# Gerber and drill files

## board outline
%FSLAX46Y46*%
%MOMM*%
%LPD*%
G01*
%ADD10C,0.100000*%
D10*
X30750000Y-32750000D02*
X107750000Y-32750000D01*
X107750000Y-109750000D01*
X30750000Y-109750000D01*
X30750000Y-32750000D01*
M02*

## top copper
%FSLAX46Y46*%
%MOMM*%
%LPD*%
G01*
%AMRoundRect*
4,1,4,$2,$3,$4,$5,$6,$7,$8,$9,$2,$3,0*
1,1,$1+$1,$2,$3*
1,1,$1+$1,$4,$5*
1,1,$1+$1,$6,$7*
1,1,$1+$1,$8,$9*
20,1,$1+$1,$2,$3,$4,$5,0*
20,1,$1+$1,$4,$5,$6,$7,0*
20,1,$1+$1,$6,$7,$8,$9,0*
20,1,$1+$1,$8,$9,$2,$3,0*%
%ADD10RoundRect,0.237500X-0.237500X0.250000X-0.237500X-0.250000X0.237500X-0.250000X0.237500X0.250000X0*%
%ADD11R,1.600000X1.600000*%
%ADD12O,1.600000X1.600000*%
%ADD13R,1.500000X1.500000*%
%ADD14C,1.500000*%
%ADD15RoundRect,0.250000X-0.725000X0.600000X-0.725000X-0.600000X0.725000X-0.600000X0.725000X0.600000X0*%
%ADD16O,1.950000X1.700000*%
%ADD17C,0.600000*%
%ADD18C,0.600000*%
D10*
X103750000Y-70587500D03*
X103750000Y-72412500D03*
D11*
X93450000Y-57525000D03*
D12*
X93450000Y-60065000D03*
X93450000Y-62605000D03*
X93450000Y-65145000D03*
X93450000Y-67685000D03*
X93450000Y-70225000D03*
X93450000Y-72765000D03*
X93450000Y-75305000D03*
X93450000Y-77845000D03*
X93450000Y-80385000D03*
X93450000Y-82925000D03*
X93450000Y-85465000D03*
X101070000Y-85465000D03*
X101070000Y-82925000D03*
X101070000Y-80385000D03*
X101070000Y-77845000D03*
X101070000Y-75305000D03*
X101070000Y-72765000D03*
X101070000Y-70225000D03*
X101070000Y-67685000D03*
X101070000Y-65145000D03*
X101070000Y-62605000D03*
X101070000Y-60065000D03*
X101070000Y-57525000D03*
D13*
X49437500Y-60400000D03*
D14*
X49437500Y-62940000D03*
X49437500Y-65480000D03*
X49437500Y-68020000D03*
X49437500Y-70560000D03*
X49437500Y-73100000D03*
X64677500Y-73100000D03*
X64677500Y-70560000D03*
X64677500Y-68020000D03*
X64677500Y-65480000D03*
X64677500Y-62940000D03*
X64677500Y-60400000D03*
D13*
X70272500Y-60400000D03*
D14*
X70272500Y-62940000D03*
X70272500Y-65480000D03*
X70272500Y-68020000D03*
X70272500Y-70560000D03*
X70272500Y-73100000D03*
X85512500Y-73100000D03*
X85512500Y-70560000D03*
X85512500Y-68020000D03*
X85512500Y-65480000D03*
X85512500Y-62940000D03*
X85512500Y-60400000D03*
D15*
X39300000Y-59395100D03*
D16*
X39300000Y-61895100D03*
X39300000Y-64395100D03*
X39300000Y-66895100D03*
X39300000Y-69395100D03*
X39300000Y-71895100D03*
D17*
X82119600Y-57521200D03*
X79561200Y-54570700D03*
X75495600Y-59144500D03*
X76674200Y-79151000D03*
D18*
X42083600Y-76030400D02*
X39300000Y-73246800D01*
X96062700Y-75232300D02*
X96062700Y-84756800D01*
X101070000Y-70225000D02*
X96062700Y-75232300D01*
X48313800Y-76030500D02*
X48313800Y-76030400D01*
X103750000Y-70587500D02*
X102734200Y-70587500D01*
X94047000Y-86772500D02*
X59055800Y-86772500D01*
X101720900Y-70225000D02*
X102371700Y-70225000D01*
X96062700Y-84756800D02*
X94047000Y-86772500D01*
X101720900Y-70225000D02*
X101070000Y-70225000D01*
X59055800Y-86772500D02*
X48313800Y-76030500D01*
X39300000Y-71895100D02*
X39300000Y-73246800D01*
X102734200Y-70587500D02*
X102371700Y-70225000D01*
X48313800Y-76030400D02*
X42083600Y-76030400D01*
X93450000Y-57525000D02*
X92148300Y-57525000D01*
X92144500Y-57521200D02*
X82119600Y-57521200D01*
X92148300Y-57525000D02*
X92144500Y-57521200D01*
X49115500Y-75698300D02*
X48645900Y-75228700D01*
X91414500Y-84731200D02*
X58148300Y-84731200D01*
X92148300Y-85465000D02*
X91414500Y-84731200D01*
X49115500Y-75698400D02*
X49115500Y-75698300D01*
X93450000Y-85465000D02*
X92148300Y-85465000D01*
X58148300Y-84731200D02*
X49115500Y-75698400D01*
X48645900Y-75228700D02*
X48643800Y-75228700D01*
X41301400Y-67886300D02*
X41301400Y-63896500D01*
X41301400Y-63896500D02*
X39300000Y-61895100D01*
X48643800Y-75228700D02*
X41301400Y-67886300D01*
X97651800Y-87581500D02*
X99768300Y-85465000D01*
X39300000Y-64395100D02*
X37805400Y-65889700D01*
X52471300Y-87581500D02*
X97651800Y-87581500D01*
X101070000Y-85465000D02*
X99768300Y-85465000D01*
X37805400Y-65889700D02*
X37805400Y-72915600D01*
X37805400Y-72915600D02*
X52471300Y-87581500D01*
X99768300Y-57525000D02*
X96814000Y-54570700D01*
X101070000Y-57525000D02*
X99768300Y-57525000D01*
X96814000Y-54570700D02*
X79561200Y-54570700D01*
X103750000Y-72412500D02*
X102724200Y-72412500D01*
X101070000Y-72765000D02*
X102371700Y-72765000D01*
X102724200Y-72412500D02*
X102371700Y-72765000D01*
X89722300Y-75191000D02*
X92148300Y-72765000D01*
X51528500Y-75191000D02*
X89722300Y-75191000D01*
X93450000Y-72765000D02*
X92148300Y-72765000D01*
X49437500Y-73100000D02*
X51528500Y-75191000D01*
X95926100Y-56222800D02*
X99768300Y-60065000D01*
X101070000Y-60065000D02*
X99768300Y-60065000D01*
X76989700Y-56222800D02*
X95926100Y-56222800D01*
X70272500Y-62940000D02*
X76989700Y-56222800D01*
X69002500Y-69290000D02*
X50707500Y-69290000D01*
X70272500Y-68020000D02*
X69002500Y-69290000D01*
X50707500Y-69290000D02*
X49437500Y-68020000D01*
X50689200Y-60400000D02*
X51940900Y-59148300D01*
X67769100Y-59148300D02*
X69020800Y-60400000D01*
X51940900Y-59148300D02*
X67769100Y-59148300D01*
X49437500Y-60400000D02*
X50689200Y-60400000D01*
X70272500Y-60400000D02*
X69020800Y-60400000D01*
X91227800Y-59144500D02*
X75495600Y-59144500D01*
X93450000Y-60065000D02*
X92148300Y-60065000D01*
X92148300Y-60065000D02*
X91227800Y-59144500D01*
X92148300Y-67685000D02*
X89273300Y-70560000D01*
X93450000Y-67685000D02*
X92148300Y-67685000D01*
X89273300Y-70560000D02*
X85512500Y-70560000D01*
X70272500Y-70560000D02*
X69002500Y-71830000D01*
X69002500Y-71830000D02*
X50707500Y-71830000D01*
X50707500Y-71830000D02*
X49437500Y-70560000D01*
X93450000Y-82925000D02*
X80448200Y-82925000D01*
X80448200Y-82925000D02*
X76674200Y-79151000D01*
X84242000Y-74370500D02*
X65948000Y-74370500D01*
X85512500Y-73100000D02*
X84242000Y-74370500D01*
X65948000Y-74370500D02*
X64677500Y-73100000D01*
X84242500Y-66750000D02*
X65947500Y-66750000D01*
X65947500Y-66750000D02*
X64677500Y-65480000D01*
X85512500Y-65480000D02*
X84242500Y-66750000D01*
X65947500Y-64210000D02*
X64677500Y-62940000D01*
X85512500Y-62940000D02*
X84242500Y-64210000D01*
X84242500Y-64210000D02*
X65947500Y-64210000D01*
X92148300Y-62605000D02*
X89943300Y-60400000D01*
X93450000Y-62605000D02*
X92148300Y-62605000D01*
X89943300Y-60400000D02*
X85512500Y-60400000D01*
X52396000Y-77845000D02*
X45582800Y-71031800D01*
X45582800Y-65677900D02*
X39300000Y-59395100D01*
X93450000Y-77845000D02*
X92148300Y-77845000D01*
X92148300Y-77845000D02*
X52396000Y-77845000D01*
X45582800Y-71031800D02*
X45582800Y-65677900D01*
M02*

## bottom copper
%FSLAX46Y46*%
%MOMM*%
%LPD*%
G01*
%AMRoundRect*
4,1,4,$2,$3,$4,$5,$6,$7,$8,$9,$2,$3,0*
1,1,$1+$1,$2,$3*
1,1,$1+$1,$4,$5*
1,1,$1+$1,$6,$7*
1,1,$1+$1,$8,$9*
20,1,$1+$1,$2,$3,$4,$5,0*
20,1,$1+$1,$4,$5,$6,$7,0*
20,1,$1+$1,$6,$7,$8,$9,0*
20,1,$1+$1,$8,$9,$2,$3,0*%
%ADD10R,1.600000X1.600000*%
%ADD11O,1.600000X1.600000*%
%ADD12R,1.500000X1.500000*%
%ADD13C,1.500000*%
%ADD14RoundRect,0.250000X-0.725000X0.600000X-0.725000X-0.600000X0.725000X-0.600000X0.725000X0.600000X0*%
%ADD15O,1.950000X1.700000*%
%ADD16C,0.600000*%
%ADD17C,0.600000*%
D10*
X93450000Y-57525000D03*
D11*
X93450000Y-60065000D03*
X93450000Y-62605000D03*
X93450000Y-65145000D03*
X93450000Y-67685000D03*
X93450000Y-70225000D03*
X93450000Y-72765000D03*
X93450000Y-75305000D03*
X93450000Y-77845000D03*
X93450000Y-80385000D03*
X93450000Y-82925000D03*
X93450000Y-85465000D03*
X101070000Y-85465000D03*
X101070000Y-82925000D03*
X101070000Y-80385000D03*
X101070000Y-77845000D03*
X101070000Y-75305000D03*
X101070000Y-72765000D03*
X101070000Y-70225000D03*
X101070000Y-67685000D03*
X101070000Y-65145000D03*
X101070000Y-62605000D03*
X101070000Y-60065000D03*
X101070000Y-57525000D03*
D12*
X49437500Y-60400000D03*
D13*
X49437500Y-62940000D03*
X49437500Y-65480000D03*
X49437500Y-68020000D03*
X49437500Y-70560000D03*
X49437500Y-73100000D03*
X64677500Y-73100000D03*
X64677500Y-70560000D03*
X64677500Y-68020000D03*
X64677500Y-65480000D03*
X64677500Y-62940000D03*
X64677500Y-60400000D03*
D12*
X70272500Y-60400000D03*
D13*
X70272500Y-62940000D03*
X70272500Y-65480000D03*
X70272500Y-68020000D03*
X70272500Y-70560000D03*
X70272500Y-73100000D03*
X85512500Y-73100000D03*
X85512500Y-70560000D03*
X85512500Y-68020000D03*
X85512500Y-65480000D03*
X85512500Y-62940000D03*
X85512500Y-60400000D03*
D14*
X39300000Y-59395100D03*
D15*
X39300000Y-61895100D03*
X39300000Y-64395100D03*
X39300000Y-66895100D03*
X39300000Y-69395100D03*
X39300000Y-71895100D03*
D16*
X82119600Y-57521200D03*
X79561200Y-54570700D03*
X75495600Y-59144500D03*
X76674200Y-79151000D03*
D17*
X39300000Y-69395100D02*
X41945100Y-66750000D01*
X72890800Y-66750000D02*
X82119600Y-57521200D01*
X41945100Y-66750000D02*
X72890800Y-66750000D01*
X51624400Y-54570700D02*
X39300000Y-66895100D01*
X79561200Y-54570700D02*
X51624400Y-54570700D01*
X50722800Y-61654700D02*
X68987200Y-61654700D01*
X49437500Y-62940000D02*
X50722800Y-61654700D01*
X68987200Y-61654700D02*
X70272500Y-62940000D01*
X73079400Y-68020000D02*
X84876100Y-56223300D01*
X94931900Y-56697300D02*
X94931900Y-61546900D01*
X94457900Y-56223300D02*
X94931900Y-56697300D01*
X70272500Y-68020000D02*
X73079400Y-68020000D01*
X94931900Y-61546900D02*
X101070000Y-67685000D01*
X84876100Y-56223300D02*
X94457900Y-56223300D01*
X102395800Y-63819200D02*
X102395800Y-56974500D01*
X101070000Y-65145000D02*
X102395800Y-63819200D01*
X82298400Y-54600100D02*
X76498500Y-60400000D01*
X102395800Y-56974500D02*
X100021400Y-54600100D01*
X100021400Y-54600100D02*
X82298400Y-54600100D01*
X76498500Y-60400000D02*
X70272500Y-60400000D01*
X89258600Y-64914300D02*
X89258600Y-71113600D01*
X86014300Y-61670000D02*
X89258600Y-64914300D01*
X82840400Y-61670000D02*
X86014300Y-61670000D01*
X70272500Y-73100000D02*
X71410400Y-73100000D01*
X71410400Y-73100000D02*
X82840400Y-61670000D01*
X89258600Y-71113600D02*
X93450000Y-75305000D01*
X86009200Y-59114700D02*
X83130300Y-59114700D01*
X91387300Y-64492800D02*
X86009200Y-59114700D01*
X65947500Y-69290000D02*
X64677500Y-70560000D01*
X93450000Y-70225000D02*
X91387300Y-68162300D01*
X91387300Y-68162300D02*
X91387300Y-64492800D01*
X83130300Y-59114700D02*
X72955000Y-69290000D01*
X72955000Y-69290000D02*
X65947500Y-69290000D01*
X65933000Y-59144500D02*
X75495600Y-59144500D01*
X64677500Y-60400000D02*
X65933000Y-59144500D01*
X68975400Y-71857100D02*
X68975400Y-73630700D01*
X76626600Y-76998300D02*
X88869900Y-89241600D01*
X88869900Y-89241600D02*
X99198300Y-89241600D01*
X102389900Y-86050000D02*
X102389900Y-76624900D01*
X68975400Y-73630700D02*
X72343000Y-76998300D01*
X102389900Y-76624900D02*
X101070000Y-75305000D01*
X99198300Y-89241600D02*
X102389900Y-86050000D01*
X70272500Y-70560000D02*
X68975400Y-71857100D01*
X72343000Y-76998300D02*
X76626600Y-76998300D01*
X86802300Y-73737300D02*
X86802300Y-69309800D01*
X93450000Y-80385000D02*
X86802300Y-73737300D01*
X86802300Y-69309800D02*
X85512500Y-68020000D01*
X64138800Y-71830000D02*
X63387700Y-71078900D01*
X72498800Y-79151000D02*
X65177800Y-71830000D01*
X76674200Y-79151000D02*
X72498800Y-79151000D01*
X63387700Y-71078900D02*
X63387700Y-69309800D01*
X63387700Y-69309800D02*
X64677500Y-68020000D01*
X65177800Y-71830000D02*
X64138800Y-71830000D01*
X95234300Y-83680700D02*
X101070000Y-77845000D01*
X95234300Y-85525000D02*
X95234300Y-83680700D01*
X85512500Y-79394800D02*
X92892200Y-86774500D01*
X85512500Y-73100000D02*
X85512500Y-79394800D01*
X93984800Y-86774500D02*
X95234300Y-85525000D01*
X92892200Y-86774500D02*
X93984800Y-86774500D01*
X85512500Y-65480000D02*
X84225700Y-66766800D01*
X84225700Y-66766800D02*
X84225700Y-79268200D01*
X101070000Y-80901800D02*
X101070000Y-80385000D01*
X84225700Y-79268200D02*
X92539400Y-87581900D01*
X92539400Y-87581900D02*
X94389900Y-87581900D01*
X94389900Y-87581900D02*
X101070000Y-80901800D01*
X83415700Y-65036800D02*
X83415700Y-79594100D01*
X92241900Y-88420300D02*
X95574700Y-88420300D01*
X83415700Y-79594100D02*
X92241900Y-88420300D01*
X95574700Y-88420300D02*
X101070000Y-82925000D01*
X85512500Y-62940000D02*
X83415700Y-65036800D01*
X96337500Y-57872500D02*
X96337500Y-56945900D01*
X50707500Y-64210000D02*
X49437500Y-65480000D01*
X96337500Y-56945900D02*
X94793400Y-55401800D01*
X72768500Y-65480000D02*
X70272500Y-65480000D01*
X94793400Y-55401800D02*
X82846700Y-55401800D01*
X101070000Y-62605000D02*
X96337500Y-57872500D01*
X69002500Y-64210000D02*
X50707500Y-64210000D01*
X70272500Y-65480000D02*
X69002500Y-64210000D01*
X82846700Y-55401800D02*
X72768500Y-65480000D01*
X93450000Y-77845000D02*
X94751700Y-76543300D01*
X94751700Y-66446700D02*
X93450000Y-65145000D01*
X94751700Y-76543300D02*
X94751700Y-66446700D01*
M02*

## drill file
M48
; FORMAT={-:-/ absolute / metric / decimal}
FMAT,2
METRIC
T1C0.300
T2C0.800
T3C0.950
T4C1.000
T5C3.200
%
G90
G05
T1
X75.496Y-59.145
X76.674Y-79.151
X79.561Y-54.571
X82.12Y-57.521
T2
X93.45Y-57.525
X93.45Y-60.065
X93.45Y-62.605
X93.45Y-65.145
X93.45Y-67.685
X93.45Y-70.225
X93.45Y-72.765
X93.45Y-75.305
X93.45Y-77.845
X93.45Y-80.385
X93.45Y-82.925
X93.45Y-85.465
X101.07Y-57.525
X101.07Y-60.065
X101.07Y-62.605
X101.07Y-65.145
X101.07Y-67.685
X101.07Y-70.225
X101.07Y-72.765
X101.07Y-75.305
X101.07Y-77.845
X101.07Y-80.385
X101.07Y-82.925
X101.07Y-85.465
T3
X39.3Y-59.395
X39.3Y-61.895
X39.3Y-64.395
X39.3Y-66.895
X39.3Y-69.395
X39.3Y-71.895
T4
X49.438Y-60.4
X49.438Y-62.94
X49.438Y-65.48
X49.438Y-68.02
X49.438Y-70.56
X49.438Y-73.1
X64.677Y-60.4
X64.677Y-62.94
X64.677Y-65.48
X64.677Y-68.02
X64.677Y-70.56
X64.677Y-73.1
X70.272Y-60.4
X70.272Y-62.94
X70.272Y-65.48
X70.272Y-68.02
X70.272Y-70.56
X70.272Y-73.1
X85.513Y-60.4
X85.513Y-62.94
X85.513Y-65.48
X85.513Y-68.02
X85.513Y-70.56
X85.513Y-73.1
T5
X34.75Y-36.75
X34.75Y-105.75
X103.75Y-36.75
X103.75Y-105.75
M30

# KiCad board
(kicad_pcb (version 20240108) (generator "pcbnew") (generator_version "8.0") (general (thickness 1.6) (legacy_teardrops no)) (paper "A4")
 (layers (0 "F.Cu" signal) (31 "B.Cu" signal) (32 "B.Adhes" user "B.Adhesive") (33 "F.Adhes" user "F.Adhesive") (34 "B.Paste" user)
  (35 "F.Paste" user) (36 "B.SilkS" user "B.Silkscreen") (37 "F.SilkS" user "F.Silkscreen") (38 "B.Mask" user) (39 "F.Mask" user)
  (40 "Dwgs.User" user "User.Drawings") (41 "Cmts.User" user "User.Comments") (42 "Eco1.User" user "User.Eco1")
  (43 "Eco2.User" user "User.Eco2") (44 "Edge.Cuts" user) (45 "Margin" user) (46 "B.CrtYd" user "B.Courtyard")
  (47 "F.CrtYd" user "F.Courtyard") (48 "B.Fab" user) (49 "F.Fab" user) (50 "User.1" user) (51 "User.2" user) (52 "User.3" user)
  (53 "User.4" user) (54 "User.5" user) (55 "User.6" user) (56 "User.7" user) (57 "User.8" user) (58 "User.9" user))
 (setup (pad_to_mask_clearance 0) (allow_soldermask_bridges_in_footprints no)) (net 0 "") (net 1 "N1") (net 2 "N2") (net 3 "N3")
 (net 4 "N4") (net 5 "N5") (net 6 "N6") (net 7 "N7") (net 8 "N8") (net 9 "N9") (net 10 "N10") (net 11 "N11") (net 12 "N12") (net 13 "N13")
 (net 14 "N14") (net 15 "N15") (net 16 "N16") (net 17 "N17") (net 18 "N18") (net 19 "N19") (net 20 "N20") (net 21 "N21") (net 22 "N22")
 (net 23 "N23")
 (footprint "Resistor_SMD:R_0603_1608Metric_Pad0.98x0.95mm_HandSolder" (layer "F.Cu") (at 103.75 71.5 -90)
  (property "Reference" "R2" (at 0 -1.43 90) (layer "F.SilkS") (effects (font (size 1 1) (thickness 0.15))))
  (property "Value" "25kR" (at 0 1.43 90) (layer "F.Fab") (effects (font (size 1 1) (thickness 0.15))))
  (pad "1" smd roundrect (at -0.9125 0 270) (size 0.975 0.95) (layers "F.Cu" "F.Paste" "F.Mask") (roundrect_rratio 0.25) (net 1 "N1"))
  (pad "2" smd roundrect (at 0.9125 0 270) (size 0.975 0.95) (layers "F.Cu" "F.Paste" "F.Mask") (roundrect_rratio 0.25) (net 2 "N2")))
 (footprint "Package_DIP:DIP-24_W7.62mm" (layer "F.Cu") (at 93.45 57.525)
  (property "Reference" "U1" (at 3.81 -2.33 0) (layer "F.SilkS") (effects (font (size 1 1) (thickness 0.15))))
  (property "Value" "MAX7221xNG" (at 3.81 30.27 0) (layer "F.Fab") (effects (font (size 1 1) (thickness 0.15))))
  (pad "1" thru_hole rect (at 0 0) (size 1.6 1.6) (drill 0.8) (layers "*.Cu" "*.Mask") (remove_unused_layers no) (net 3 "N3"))
  (pad "2" thru_hole oval (at 0 2.54) (size 1.6 1.6) (drill 0.8) (layers "*.Cu" "*.Mask") (remove_unused_layers no) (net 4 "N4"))
  (pad "3" thru_hole oval (at 0 5.08) (size 1.6 1.6) (drill 0.8) (layers "*.Cu" "*.Mask") (remove_unused_layers no) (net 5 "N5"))
  (pad "4" thru_hole oval (at 0 7.62) (size 1.6 1.6) (drill 0.8) (layers "*.Cu" "*.Mask") (remove_unused_layers no) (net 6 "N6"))
  (pad "5" thru_hole oval (at 0 10.16) (size 1.6 1.6) (drill 0.8) (layers "*.Cu" "*.Mask") (remove_unused_layers no) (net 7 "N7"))
  (pad "6" thru_hole oval (at 0 12.7) (size 1.6 1.6) (drill 0.8) (layers "*.Cu" "*.Mask") (remove_unused_layers no) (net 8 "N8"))
  (pad "7" thru_hole oval (at 0 15.24) (size 1.6 1.6) (drill 0.8) (layers "*.Cu" "*.Mask") (remove_unused_layers no) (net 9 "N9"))
  (pad "8" thru_hole oval (at 0 17.78) (size 1.6 1.6) (drill 0.8) (layers "*.Cu" "*.Mask") (remove_unused_layers no) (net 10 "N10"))
  (pad "9" thru_hole oval (at 0 20.32) (size 1.6 1.6) (drill 0.8) (layers "*.Cu" "*.Mask") (remove_unused_layers no) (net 6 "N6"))
  (pad "10" thru_hole oval (at 0 22.86) (size 1.6 1.6) (drill 0.8) (layers "*.Cu" "*.Mask") (remove_unused_layers no) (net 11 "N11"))
  (pad "11" thru_hole oval (at 0 25.4) (size 1.6 1.6) (drill 0.8) (layers "*.Cu" "*.Mask") (remove_unused_layers no) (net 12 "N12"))
  (pad "12" thru_hole oval (at 0 27.94) (size 1.6 1.6) (drill 0.8) (layers "*.Cu" "*.Mask") (remove_unused_layers no) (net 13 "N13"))
  (pad "13" thru_hole oval (at 7.62 27.94) (size 1.6 1.6) (drill 0.8) (layers "*.Cu" "*.Mask") (remove_unused_layers no) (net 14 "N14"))
  (pad "14" thru_hole oval (at 7.62 25.4) (size 1.6 1.6) (drill 0.8) (layers "*.Cu" "*.Mask") (remove_unused_layers no) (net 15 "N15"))
  (pad "15" thru_hole oval (at 7.62 22.86) (size 1.6 1.6) (drill 0.8) (layers "*.Cu" "*.Mask") (remove_unused_layers no) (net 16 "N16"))
  (pad "16" thru_hole oval (at 7.62 20.32) (size 1.6 1.6) (drill 0.8) (layers "*.Cu" "*.Mask") (remove_unused_layers no) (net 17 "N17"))
  (pad "17" thru_hole oval (at 7.62 17.78) (size 1.6 1.6) (drill 0.8) (layers "*.Cu" "*.Mask") (remove_unused_layers no) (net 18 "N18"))
  (pad "18" thru_hole oval (at 7.62 15.24) (size 1.6 1.6) (drill 0.8) (layers "*.Cu" "*.Mask") (remove_unused_layers no) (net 2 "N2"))
  (pad "19" thru_hole oval (at 7.62 12.7) (size 1.6 1.6) (drill 0.8) (layers "*.Cu" "*.Mask") (remove_unused_layers no) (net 1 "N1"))
  (pad "20" thru_hole oval (at 7.62 10.16) (size 1.6 1.6) (drill 0.8) (layers "*.Cu" "*.Mask") (remove_unused_layers no) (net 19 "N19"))
  (pad "21" thru_hole oval (at 7.62 7.62) (size 1.6 1.6) (drill 0.8) (layers "*.Cu" "*.Mask") (remove_unused_layers no) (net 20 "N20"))
  (pad "22" thru_hole oval (at 7.62 5.08) (size 1.6 1.6) (drill 0.8) (layers "*.Cu" "*.Mask") (remove_unused_layers no) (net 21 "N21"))
  (pad "23" thru_hole oval (at 7.62 2.54) (size 1.6 1.6) (drill 0.8) (layers "*.Cu" "*.Mask") (remove_unused_layers no) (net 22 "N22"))
  (pad "24" thru_hole oval (at 7.62 0) (size 1.6 1.6) (drill 0.8) (layers "*.Cu" "*.Mask") (remove_unused_layers no) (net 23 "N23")))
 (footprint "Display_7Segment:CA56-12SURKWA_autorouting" (layer "F.Cu") (at 49.4375 60.4)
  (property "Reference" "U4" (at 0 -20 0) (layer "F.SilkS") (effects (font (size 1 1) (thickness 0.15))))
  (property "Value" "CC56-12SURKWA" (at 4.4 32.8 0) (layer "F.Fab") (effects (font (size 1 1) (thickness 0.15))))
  (pad "1" thru_hole rect (at 0 0) (size 1.5 1.5) (drill 1) (layers "*.Cu" "*.Mask") (remove_unused_layers no) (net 20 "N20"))
  (pad "2" thru_hole circle (at 0 2.54) (size 1.5 1.5) (drill 1) (layers "*.Cu" "*.Mask") (remove_unused_layers no) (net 22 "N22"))
  (pad "3" thru_hole circle (at 0 5.08) (size 1.5 1.5) (drill 1) (layers "*.Cu" "*.Mask") (remove_unused_layers no) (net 21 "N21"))
  (pad "4" thru_hole circle (at 0 7.62) (size 1.5 1.5) (drill 1) (layers "*.Cu" "*.Mask") (remove_unused_layers no) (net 19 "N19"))
  (pad "5" thru_hole circle (at 0 10.16) (size 1.5 1.5) (drill 1) (layers "*.Cu" "*.Mask") (remove_unused_layers no) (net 18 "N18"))
  (pad "6" thru_hole circle (at 0 12.7) (size 1.5 1.5) (drill 1) (layers "*.Cu" "*.Mask") (remove_unused_layers no) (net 9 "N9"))
  (pad "7" thru_hole circle (at 15.24 12.7) (size 1.5 1.5) (drill 1) (layers "*.Cu" "*.Mask") (remove_unused_layers no) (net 17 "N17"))
  (pad "8" thru_hole circle (at 15.24 10.16) (size 1.5 1.5) (drill 1) (layers "*.Cu" "*.Mask") (remove_unused_layers no) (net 8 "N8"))
  (pad "9" thru_hole circle (at 15.24 7.62) (size 1.5 1.5) (drill 1) (layers "*.Cu" "*.Mask") (remove_unused_layers no) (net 12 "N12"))
  (pad "10" thru_hole circle (at 15.24 5.08) (size 1.5 1.5) (drill 1) (layers "*.Cu" "*.Mask") (remove_unused_layers no) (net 16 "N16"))
  (pad "11" thru_hole circle (at 15.24 2.54) (size 1.5 1.5) (drill 1) (layers "*.Cu" "*.Mask") (remove_unused_layers no) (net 15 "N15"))
  (pad "12" thru_hole circle (at 15.24 0) (size 1.5 1.5) (drill 1) (layers "*.Cu" "*.Mask") (remove_unused_layers no) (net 4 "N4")))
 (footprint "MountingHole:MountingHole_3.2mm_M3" (layer "F.Cu") (at 34.75 36.75)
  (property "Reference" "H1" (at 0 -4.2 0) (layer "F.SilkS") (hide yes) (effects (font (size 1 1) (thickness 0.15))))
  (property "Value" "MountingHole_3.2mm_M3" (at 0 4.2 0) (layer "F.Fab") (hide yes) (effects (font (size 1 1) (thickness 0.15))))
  (pad "" np_thru_hole circle (at 0 0) (size 3.2 3.2) (drill 3.2) (layers "*.Cu" "*.Mask")))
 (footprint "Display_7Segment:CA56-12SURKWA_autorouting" (layer "F.Cu") (at 70.2725 60.4)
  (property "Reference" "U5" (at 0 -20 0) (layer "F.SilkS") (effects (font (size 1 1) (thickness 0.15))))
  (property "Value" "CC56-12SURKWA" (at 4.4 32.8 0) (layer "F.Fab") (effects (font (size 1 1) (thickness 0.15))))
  (pad "1" thru_hole rect (at 0 0) (size 1.5 1.5) (drill 1) (layers "*.Cu" "*.Mask") (remove_unused_layers no) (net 20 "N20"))
  (pad "2" thru_hole circle (at 0 2.54) (size 1.5 1.5) (drill 1) (layers "*.Cu" "*.Mask") (remove_unused_layers no) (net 22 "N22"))
  (pad "3" thru_hole circle (at 0 5.08) (size 1.5 1.5) (drill 1) (layers "*.Cu" "*.Mask") (remove_unused_layers no) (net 21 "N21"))
  (pad "4" thru_hole circle (at 0 7.62) (size 1.5 1.5) (drill 1) (layers "*.Cu" "*.Mask") (remove_unused_layers no) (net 19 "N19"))
  (pad "5" thru_hole circle (at 0 10.16) (size 1.5 1.5) (drill 1) (layers "*.Cu" "*.Mask") (remove_unused_layers no) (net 18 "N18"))
  (pad "6" thru_hole circle (at 0 12.7) (size 1.5 1.5) (drill 1) (layers "*.Cu" "*.Mask") (remove_unused_layers no) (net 10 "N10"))
  (pad "7" thru_hole circle (at 15.24 12.7) (size 1.5 1.5) (drill 1) (layers "*.Cu" "*.Mask") (remove_unused_layers no) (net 17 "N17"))
  (pad "8" thru_hole circle (at 15.24 10.16) (size 1.5 1.5) (drill 1) (layers "*.Cu" "*.Mask") (remove_unused_layers no) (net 7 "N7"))
  (pad "9" thru_hole circle (at 15.24 7.62) (size 1.5 1.5) (drill 1) (layers "*.Cu" "*.Mask") (remove_unused_layers no) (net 11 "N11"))
  (pad "10" thru_hole circle (at 15.24 5.08) (size 1.5 1.5) (drill 1) (layers "*.Cu" "*.Mask") (remove_unused_layers no) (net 16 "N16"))
  (pad "11" thru_hole circle (at 15.24 2.54) (size 1.5 1.5) (drill 1) (layers "*.Cu" "*.Mask") (remove_unused_layers no) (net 15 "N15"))
  (pad "12" thru_hole circle (at 15.24 0) (size 1.5 1.5) (drill 1) (layers "*.Cu" "*.Mask") (remove_unused_layers no) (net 5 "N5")))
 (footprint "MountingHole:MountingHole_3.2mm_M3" (layer "F.Cu") (at 103.75 36.75)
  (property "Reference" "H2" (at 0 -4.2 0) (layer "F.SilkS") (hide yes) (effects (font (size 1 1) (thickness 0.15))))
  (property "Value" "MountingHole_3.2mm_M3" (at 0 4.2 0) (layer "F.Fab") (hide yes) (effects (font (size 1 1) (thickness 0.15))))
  (pad "" np_thru_hole circle (at 0 0) (size 3.2 3.2) (drill 3.2) (layers "F&B.Cu" "*.Mask")))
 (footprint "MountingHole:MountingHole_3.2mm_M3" (layer "F.Cu") (at 34.75 105.75)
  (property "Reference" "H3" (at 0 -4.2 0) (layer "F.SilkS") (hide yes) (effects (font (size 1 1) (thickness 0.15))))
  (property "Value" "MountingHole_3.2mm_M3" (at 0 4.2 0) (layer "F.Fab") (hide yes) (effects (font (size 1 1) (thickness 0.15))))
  (pad "" np_thru_hole circle (at 0 0) (size 3.2 3.2) (drill 3.2) (layers "F&B.Cu" "*.Mask")))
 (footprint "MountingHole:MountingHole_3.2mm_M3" (layer "F.Cu") (at 103.75 105.75)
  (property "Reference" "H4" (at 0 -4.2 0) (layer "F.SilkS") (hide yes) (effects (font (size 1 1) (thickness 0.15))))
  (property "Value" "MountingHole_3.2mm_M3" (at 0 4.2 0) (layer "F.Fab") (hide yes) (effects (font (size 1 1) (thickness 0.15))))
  (pad "" np_thru_hole circle (at 0 0) (size 3.2 3.2) (drill 3.2) (layers "F&B.Cu" "*.Mask")))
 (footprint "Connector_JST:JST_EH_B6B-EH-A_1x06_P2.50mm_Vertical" (layer "F.Cu") (at 39.3 59.3951 -90)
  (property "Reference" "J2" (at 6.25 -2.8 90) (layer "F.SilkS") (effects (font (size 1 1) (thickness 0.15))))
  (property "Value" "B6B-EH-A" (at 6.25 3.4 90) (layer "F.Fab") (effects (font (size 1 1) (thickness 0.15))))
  (pad "1" thru_hole roundrect (at 0 0 270) (size 1.7 1.95) (drill 0.95) (layers "*.Cu" "*.Mask") (remove_unused_layers no)
   (roundrect_rratio 0.147059) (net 6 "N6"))
  (pad "2" thru_hole oval (at 2.5 0 270) (size 1.7 1.95) (drill 0.95) (layers "*.Cu" "*.Mask") (remove_unused_layers no) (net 13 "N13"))
  (pad "3" thru_hole oval (at 5 0 270) (size 1.7 1.95) (drill 0.95) (layers "*.Cu" "*.Mask") (remove_unused_layers no) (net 14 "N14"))
  (pad "4" thru_hole oval (at 7.5 0 270) (size 1.7 1.95) (drill 0.95) (layers "*.Cu" "*.Mask") (remove_unused_layers no) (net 23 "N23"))
  (pad "5" thru_hole oval (at 10 0 270) (size 1.7 1.95) (drill 0.95) (layers "*.Cu" "*.Mask") (remove_unused_layers no) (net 3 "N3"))
  (pad "6" thru_hole oval (at 12.5 0 270) (size 1.7 1.95) (drill 0.95) (layers "*.Cu" "*.Mask") (remove_unused_layers no) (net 1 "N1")))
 (gr_rect (start 30.75 32.75) (end 107.75 109.75) (stroke (width 0.1) (type default)) (fill none) (layer "Edge.Cuts"))
 (segment (start 42.0836 76.0304) (end 39.3 73.2468) (width 0.6) (layer "F.Cu") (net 1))
 (segment (start 96.0627 75.2323) (end 96.0627 84.7568) (width 0.6) (layer "F.Cu") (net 1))
 (segment (start 101.07 70.225) (end 96.0627 75.2323) (width 0.6) (layer "F.Cu") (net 1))
 (segment (start 48.3138 76.0305) (end 48.3138 76.0304) (width 0.6) (layer "F.Cu") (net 1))
 (segment (start 103.75 70.5875) (end 102.7342 70.5875) (width 0.6) (layer "F.Cu") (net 1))
 (segment (start 94.047 86.7725) (end 59.0558 86.7725) (width 0.6) (layer "F.Cu") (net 1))
 (segment (start 101.7209 70.225) (end 102.3717 70.225) (width 0.6) (layer "F.Cu") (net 1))
 (segment (start 96.0627 84.7568) (end 94.047 86.7725) (width 0.6) (layer "F.Cu") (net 1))
 (segment (start 101.7209 70.225) (end 101.07 70.225) (width 0.6) (layer "F.Cu") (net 1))
 (segment (start 59.0558 86.7725) (end 48.3138 76.0305) (width 0.6) (layer "F.Cu") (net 1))
 (segment (start 39.3 71.8951) (end 39.3 73.2468) (width 0.6) (layer "F.Cu") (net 1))
 (segment (start 102.7342 70.5875) (end 102.3717 70.225) (width 0.6) (layer "F.Cu") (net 1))
 (segment (start 48.3138 76.0304) (end 42.0836 76.0304) (width 0.6) (layer "F.Cu") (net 1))
 (segment (start 93.45 57.525) (end 92.1483 57.525) (width 0.6) (layer "F.Cu") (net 3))
 (segment (start 92.1445 57.5212) (end 82.1196 57.5212) (width 0.6) (layer "F.Cu") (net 3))
 (segment (start 92.1483 57.525) (end 92.1445 57.5212) (width 0.6) (layer "F.Cu") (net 3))
 (via (at 82.1196 57.5212) (size 0.6) (drill 0.3) (layers "F.Cu" "B.Cu") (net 3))
 (segment (start 39.3 69.3951) (end 41.9451 66.75) (width 0.6) (layer "B.Cu") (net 3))
 (segment (start 72.8908 66.75) (end 82.1196 57.5212) (width 0.6) (layer "B.Cu") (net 3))
 (segment (start 41.9451 66.75) (end 72.8908 66.75) (width 0.6) (layer "B.Cu") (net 3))
 (segment (start 49.1155 75.6983) (end 48.6459 75.2287) (width 0.6) (layer "F.Cu") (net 13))
 (segment (start 91.4145 84.7312) (end 58.1483 84.7312) (width 0.6) (layer "F.Cu") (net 13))
 (segment (start 92.1483 85.465) (end 91.4145 84.7312) (width 0.6) (layer "F.Cu") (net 13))
 (segment (start 49.1155 75.6984) (end 49.1155 75.6983) (width 0.6) (layer "F.Cu") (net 13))
 (segment (start 93.45 85.465) (end 92.1483 85.465) (width 0.6) (layer "F.Cu") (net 13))
 (segment (start 58.1483 84.7312) (end 49.1155 75.6984) (width 0.6) (layer "F.Cu") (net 13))
 (segment (start 48.6459 75.2287) (end 48.6438 75.2287) (width 0.6) (layer "F.Cu") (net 13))
 (segment (start 41.3014 67.8863) (end 41.3014 63.8965) (width 0.6) (layer "F.Cu") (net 13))
 (segment (start 41.3014 63.8965) (end 39.3 61.8951) (width 0.6) (layer "F.Cu") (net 13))
 (segment (start 48.6438 75.2287) (end 41.3014 67.8863) (width 0.6) (layer "F.Cu") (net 13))
 (segment (start 97.6518 87.5815) (end 99.7683 85.465) (width 0.6) (layer "F.Cu") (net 14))
 (segment (start 39.3 64.3951) (end 37.8054 65.8897) (width 0.6) (layer "F.Cu") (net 14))
 (segment (start 52.4713 87.5815) (end 97.6518 87.5815) (width 0.6) (layer "F.Cu") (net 14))
 (segment (start 101.07 85.465) (end 99.7683 85.465) (width 0.6) (layer "F.Cu") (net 14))
 (segment (start 37.8054 65.8897) (end 37.8054 72.9156) (width 0.6) (layer "F.Cu") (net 14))
 (segment (start 37.8054 72.9156) (end 52.4713 87.5815) (width 0.6) (layer "F.Cu") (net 14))
 (segment (start 99.7683 57.525) (end 96.814 54.5707) (width 0.6) (layer "F.Cu") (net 23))
 (segment (start 101.07 57.525) (end 99.7683 57.525) (width 0.6) (layer "F.Cu") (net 23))
 (segment (start 96.814 54.5707) (end 79.5612 54.5707) (width 0.6) (layer "F.Cu") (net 23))
 (via (at 79.5612 54.5707) (size 0.6) (drill 0.3) (layers "F.Cu" "B.Cu") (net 23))
 (segment (start 51.6244 54.5707) (end 39.3 66.8951) (width 0.6) (layer "B.Cu") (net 23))
 (segment (start 79.5612 54.5707) (end 51.6244 54.5707) (width 0.6) (layer "B.Cu") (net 23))
 (segment (start 103.75 72.4125) (end 102.7242 72.4125) (width 0.6) (layer "F.Cu") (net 2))
 (segment (start 101.07 72.765) (end 102.3717 72.765) (width 0.6) (layer "F.Cu") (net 2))
 (segment (start 102.7242 72.4125) (end 102.3717 72.765) (width 0.6) (layer "F.Cu") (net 2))
 (segment (start 89.7223 75.191) (end 92.1483 72.765) (width 0.6) (layer "F.Cu") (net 9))
 (segment (start 51.5285 75.191) (end 89.7223 75.191) (width 0.6) (layer "F.Cu") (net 9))
 (segment (start 93.45 72.765) (end 92.1483 72.765) (width 0.6) (layer "F.Cu") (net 9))
 (segment (start 49.4375 73.1) (end 51.5285 75.191) (width 0.6) (layer "F.Cu") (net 9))
 (segment (start 95.9261 56.2228) (end 99.7683 60.065) (width 0.6) (layer "F.Cu") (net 22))
 (segment (start 101.07 60.065) (end 99.7683 60.065) (width 0.6) (layer "F.Cu") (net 22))
 (segment (start 76.9897 56.2228) (end 95.9261 56.2228) (width 0.6) (layer "F.Cu") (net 22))
 (segment (start 70.2725 62.94) (end 76.9897 56.2228) (width 0.6) (layer "F.Cu") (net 22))
 (segment (start 50.7228 61.6547) (end 68.9872 61.6547) (width 0.6) (layer "B.Cu") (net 22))
 (segment (start 49.4375 62.94) (end 50.7228 61.6547) (width 0.6) (layer "B.Cu") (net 22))
 (segment (start 68.9872 61.6547) (end 70.2725 62.94) (width 0.6) (layer "B.Cu") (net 22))
 (segment (start 69.0025 69.29) (end 50.7075 69.29) (width 0.6) (layer "F.Cu") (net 19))
 (segment (start 70.2725 68.02) (end 69.0025 69.29) (width 0.6) (layer "F.Cu") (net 19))
 (segment (start 50.7075 69.29) (end 49.4375 68.02) (width 0.6) (layer "F.Cu") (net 19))
 (segment (start 73.0794 68.02) (end 84.8761 56.2233) (width 0.6) (layer "B.Cu") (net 19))
 (segment (start 94.9319 56.6973) (end 94.9319 61.5469) (width 0.6) (layer "B.Cu") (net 19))
 (segment (start 94.4579 56.2233) (end 94.9319 56.6973) (width 0.6) (layer "B.Cu") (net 19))
 (segment (start 70.2725 68.02) (end 73.0794 68.02) (width 0.6) (layer "B.Cu") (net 19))
 (segment (start 94.9319 61.5469) (end 101.07 67.685) (width 0.6) (layer "B.Cu") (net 19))
 (segment (start 84.8761 56.2233) (end 94.4579 56.2233) (width 0.6) (layer "B.Cu") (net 19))
 (segment (start 50.6892 60.4) (end 51.9409 59.1483) (width 0.6) (layer "F.Cu") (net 20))
 (segment (start 67.7691 59.1483) (end 69.0208 60.4) (width 0.6) (layer "F.Cu") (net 20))
 (segment (start 51.9409 59.1483) (end 67.7691 59.1483) (width 0.6) (layer "F.Cu") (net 20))
 (segment (start 49.4375 60.4) (end 50.6892 60.4) (width 0.6) (layer "F.Cu") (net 20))
 (segment (start 70.2725 60.4) (end 69.0208 60.4) (width 0.6) (layer "F.Cu") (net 20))
 (segment (start 102.3958 63.8192) (end 102.3958 56.9745) (width 0.6) (layer "B.Cu") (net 20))
 (segment (start 101.07 65.145) (end 102.3958 63.8192) (width 0.6) (layer "B.Cu") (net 20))
 (segment (start 82.2984 54.6001) (end 76.4985 60.4) (width 0.6) (layer "B.Cu") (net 20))
 (segment (start 102.3958 56.9745) (end 100.0214 54.6001) (width 0.6) (layer "B.Cu") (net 20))
 (segment (start 100.0214 54.6001) (end 82.2984 54.6001) (width 0.6) (layer "B.Cu") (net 20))
 (segment (start 76.4985 60.4) (end 70.2725 60.4) (width 0.6) (layer "B.Cu") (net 20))
 (segment (start 89.2586 64.9143) (end 89.2586 71.1136) (width 0.6) (layer "B.Cu") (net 10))
 (segment (start 86.0143 61.67) (end 89.2586 64.9143) (width 0.6) (layer "B.Cu") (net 10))
 (segment (start 82.8404 61.67) (end 86.0143 61.67) (width 0.6) (layer "B.Cu") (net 10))
 (segment (start 70.2725 73.1) (end 71.4104 73.1) (width 0.6) (layer "B.Cu") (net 10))
 (segment (start 71.4104 73.1) (end 82.8404 61.67) (width 0.6) (layer "B.Cu") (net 10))
 (segment (start 89.2586 71.1136) (end 93.45 75.305) (width 0.6) (layer "B.Cu") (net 10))
 (segment (start 86.0092 59.1147) (end 83.1303 59.1147) (width 0.6) (layer "B.Cu") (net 8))
 (segment (start 91.3873 64.4928) (end 86.0092 59.1147) (width 0.6) (layer "B.Cu") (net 8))
 (segment (start 65.9475 69.29) (end 64.6775 70.56) (width 0.6) (layer "B.Cu") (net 8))
 (segment (start 93.45 70.225) (end 91.3873 68.1623) (width 0.6) (layer "B.Cu") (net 8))
 (segment (start 91.3873 68.1623) (end 91.3873 64.4928) (width 0.6) (layer "B.Cu") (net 8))
 (segment (start 83.1303 59.1147) (end 72.955 69.29) (width 0.6) (layer "B.Cu") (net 8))
 (segment (start 72.955 69.29) (end 65.9475 69.29) (width 0.6) (layer "B.Cu") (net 8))
 (segment (start 91.2278 59.1445) (end 75.4956 59.1445) (width 0.6) (layer "F.Cu") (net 4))
 (segment (start 93.45 60.065) (end 92.1483 60.065) (width 0.6) (layer "F.Cu") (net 4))
 (segment (start 92.1483 60.065) (end 91.2278 59.1445) (width 0.6) (layer "F.Cu") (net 4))
 (via (at 75.4956 59.1445) (size 0.6) (drill 0.3) (layers "F.Cu" "B.Cu") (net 4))
 (segment (start 65.933 59.1445) (end 75.4956 59.1445) (width 0.6) (layer "B.Cu") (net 4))
 (segment (start 64.6775 60.4) (end 65.933 59.1445) (width 0.6) (layer "B.Cu") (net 4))
 (segment (start 92.1483 67.685) (end 89.2733 70.56) (width 0.6) (layer "F.Cu") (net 7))
 (segment (start 93.45 67.685) (end 92.1483 67.685) (width 0.6) (layer "F.Cu") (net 7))
 (segment (start 89.2733 70.56) (end 85.5125 70.56) (width 0.6) (layer "F.Cu") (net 7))
 (segment (start 70.2725 70.56) (end 69.0025 71.83) (width 0.6) (layer "F.Cu") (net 18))
 (segment (start 69.0025 71.83) (end 50.7075 71.83) (width 0.6) (layer "F.Cu") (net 18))
 (segment (start 50.7075 71.83) (end 49.4375 70.56) (width 0.6) (layer "F.Cu") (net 18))
 (segment (start 68.9754 71.8571) (end 68.9754 73.6307) (width 0.6) (layer "B.Cu") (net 18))
 (segment (start 76.6266 76.9983) (end 88.8699 89.2416) (width 0.6) (layer "B.Cu") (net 18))
 (segment (start 88.8699 89.2416) (end 99.1983 89.2416) (width 0.6) (layer "B.Cu") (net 18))
 (segment (start 102.3899 86.05) (end 102.3899 76.6249) (width 0.6) (layer "B.Cu") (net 18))
 (segment (start 68.9754 73.6307) (end 72.343 76.9983) (width 0.6) (layer "B.Cu") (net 18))
 (segment (start 102.3899 76.6249) (end 101.07 75.305) (width 0.6) (layer "B.Cu") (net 18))
 (segment (start 99.1983 89.2416) (end 102.3899 86.05) (width 0.6) (layer "B.Cu") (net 18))
 (segment (start 70.2725 70.56) (end 68.9754 71.8571) (width 0.6) (layer "B.Cu") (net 18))
 (segment (start 72.343 76.9983) (end 76.6266 76.9983) (width 0.6) (layer "B.Cu") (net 18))
 (segment (start 86.8023 73.7373) (end 86.8023 69.3098) (width 0.6) (layer "B.Cu") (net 11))
 (segment (start 93.45 80.385) (end 86.8023 73.7373) (width 0.6) (layer "B.Cu") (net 11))
 (segment (start 86.8023 69.3098) (end 85.5125 68.02) (width 0.6) (layer "B.Cu") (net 11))
 (segment (start 93.45 82.925) (end 80.4482 82.925) (width 0.6) (layer "F.Cu") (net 12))
 (segment (start 80.4482 82.925) (end 76.6742 79.151) (width 0.6) (layer "F.Cu") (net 12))
 (via (at 76.6742 79.151) (size 0.6) (drill 0.3) (layers "F.Cu" "B.Cu") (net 12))
 (segment (start 64.1388 71.83) (end 63.3877 71.0789) (width 0.6) (layer "B.Cu") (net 12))
 (segment (start 72.4988 79.151) (end 65.1778 71.83) (width 0.6) (layer "B.Cu") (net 12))
 (segment (start 76.6742 79.151) (end 72.4988 79.151) (width 0.6) (layer "B.Cu") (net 12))
 (segment (start 63.3877 71.0789) (end 63.3877 69.3098) (width 0.6) (layer "B.Cu") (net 12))
 (segment (start 63.3877 69.3098) (end 64.6775 68.02) (width 0.6) (layer "B.Cu") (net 12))
 (segment (start 65.1778 71.83) (end 64.1388 71.83) (width 0.6) (layer "B.Cu") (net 12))
 (segment (start 84.242 74.3705) (end 65.948 74.3705) (width 0.6) (layer "F.Cu") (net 17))
 (segment (start 85.5125 73.1) (end 84.242 74.3705) (width 0.6) (layer "F.Cu") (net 17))
 (segment (start 65.948 74.3705) (end 64.6775 73.1) (width 0.6) (layer "F.Cu") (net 17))
 (segment (start 95.2343 83.6807) (end 101.07 77.845) (width 0.6) (layer "B.Cu") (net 17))
 (segment (start 95.2343 85.525) (end 95.2343 83.6807) (width 0.6) (layer "B.Cu") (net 17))
 (segment (start 85.5125 79.3948) (end 92.8922 86.7745) (width 0.6) (layer "B.Cu") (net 17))
 (segment (start 85.5125 73.1) (end 85.5125 79.3948) (width 0.6) (layer "B.Cu") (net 17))
 (segment (start 93.9848 86.7745) (end 95.2343 85.525) (width 0.6) (layer "B.Cu") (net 17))
 (segment (start 92.8922 86.7745) (end 93.9848 86.7745) (width 0.6) (layer "B.Cu") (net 17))
 (segment (start 84.2425 66.75) (end 65.9475 66.75) (width 0.6) (layer "F.Cu") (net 16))
 (segment (start 65.9475 66.75) (end 64.6775 65.48) (width 0.6) (layer "F.Cu") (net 16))
 (segment (start 85.5125 65.48) (end 84.2425 66.75) (width 0.6) (layer "F.Cu") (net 16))
 (segment (start 85.5125 65.48) (end 84.2257 66.7668) (width 0.6) (layer "B.Cu") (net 16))
 (segment (start 84.2257 66.7668) (end 84.2257 79.2682) (width 0.6) (layer "B.Cu") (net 16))
 (segment (start 101.07 80.9018) (end 101.07 80.385) (width 0.6) (layer "B.Cu") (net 16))
 (segment (start 84.2257 79.2682) (end 92.5394 87.5819) (width 0.6) (layer "B.Cu") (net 16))
 (segment (start 92.5394 87.5819) (end 94.3899 87.5819) (width 0.6) (layer "B.Cu") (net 16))
 (segment (start 94.3899 87.5819) (end 101.07 80.9018) (width 0.6) (layer "B.Cu") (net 16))
 (segment (start 65.9475 64.21) (end 64.6775 62.94) (width 0.6) (layer "F.Cu") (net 15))
 (segment (start 85.5125 62.94) (end 84.2425 64.21) (width 0.6) (layer "F.Cu") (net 15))
 (segment (start 84.2425 64.21) (end 65.9475 64.21) (width 0.6) (layer "F.Cu") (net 15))
 (segment (start 83.4157 65.0368) (end 83.4157 79.5941) (width 0.6) (layer "B.Cu") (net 15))
 (segment (start 92.2419 88.4203) (end 95.5747 88.4203) (width 0.6) (layer "B.Cu") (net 15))
 (segment (start 83.4157 79.5941) (end 92.2419 88.4203) (width 0.6) (layer "B.Cu") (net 15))
 (segment (start 95.5747 88.4203) (end 101.07 82.925) (width 0.6) (layer "B.Cu") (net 15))
 (segment (start 85.5125 62.94) (end 83.4157 65.0368) (width 0.6) (layer "B.Cu") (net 15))
 (segment (start 96.3375 57.8725) (end 96.3375 56.9459) (width 0.6) (layer "B.Cu") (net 21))
 (segment (start 50.7075 64.21) (end 49.4375 65.48) (width 0.6) (layer "B.Cu") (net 21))
 (segment (start 96.3375 56.9459) (end 94.7934 55.4018) (width 0.6) (layer "B.Cu") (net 21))
 (segment (start 72.7685 65.48) (end 70.2725 65.48) (width 0.6) (layer "B.Cu") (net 21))
 (segment (start 94.7934 55.4018) (end 82.8467 55.4018) (width 0.6) (layer "B.Cu") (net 21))
 (segment (start 101.07 62.605) (end 96.3375 57.8725) (width 0.6) (layer "B.Cu") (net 21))
 (segment (start 69.0025 64.21) (end 50.7075 64.21) (width 0.6) (layer "B.Cu") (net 21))
 (segment (start 70.2725 65.48) (end 69.0025 64.21) (width 0.6) (layer "B.Cu") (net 21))
 (segment (start 82.8467 55.4018) (end 72.7685 65.48) (width 0.6) (layer "B.Cu") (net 21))
 (segment (start 92.1483 62.605) (end 89.9433 60.4) (width 0.6) (layer "F.Cu") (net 5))
 (segment (start 93.45 62.605) (end 92.1483 62.605) (width 0.6) (layer "F.Cu") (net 5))
 (segment (start 89.9433 60.4) (end 85.5125 60.4) (width 0.6) (layer "F.Cu") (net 5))
 (segment (start 52.396 77.845) (end 45.5828 71.0318) (width 0.6) (layer "F.Cu") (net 6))
 (segment (start 45.5828 65.6779) (end 39.3 59.3951) (width 0.6) (layer "F.Cu") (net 6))
 (segment (start 93.45 77.845) (end 92.1483 77.845) (width 0.6) (layer "F.Cu") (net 6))
 (segment (start 92.1483 77.845) (end 52.396 77.845) (width 0.6) (layer "F.Cu") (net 6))
 (segment (start 45.5828 71.0318) (end 45.5828 65.6779) (width 0.6) (layer "F.Cu") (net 6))
 (segment (start 93.45 77.845) (end 94.7517 76.5433) (width 0.6) (layer "B.Cu") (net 6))
 (segment (start 94.7517 66.4467) (end 93.45 65.145) (width 0.6) (layer "B.Cu") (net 6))
 (segment (start 94.7517 76.5433) (end 94.7517 66.4467) (width 0.6) (layer "B.Cu") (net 6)))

